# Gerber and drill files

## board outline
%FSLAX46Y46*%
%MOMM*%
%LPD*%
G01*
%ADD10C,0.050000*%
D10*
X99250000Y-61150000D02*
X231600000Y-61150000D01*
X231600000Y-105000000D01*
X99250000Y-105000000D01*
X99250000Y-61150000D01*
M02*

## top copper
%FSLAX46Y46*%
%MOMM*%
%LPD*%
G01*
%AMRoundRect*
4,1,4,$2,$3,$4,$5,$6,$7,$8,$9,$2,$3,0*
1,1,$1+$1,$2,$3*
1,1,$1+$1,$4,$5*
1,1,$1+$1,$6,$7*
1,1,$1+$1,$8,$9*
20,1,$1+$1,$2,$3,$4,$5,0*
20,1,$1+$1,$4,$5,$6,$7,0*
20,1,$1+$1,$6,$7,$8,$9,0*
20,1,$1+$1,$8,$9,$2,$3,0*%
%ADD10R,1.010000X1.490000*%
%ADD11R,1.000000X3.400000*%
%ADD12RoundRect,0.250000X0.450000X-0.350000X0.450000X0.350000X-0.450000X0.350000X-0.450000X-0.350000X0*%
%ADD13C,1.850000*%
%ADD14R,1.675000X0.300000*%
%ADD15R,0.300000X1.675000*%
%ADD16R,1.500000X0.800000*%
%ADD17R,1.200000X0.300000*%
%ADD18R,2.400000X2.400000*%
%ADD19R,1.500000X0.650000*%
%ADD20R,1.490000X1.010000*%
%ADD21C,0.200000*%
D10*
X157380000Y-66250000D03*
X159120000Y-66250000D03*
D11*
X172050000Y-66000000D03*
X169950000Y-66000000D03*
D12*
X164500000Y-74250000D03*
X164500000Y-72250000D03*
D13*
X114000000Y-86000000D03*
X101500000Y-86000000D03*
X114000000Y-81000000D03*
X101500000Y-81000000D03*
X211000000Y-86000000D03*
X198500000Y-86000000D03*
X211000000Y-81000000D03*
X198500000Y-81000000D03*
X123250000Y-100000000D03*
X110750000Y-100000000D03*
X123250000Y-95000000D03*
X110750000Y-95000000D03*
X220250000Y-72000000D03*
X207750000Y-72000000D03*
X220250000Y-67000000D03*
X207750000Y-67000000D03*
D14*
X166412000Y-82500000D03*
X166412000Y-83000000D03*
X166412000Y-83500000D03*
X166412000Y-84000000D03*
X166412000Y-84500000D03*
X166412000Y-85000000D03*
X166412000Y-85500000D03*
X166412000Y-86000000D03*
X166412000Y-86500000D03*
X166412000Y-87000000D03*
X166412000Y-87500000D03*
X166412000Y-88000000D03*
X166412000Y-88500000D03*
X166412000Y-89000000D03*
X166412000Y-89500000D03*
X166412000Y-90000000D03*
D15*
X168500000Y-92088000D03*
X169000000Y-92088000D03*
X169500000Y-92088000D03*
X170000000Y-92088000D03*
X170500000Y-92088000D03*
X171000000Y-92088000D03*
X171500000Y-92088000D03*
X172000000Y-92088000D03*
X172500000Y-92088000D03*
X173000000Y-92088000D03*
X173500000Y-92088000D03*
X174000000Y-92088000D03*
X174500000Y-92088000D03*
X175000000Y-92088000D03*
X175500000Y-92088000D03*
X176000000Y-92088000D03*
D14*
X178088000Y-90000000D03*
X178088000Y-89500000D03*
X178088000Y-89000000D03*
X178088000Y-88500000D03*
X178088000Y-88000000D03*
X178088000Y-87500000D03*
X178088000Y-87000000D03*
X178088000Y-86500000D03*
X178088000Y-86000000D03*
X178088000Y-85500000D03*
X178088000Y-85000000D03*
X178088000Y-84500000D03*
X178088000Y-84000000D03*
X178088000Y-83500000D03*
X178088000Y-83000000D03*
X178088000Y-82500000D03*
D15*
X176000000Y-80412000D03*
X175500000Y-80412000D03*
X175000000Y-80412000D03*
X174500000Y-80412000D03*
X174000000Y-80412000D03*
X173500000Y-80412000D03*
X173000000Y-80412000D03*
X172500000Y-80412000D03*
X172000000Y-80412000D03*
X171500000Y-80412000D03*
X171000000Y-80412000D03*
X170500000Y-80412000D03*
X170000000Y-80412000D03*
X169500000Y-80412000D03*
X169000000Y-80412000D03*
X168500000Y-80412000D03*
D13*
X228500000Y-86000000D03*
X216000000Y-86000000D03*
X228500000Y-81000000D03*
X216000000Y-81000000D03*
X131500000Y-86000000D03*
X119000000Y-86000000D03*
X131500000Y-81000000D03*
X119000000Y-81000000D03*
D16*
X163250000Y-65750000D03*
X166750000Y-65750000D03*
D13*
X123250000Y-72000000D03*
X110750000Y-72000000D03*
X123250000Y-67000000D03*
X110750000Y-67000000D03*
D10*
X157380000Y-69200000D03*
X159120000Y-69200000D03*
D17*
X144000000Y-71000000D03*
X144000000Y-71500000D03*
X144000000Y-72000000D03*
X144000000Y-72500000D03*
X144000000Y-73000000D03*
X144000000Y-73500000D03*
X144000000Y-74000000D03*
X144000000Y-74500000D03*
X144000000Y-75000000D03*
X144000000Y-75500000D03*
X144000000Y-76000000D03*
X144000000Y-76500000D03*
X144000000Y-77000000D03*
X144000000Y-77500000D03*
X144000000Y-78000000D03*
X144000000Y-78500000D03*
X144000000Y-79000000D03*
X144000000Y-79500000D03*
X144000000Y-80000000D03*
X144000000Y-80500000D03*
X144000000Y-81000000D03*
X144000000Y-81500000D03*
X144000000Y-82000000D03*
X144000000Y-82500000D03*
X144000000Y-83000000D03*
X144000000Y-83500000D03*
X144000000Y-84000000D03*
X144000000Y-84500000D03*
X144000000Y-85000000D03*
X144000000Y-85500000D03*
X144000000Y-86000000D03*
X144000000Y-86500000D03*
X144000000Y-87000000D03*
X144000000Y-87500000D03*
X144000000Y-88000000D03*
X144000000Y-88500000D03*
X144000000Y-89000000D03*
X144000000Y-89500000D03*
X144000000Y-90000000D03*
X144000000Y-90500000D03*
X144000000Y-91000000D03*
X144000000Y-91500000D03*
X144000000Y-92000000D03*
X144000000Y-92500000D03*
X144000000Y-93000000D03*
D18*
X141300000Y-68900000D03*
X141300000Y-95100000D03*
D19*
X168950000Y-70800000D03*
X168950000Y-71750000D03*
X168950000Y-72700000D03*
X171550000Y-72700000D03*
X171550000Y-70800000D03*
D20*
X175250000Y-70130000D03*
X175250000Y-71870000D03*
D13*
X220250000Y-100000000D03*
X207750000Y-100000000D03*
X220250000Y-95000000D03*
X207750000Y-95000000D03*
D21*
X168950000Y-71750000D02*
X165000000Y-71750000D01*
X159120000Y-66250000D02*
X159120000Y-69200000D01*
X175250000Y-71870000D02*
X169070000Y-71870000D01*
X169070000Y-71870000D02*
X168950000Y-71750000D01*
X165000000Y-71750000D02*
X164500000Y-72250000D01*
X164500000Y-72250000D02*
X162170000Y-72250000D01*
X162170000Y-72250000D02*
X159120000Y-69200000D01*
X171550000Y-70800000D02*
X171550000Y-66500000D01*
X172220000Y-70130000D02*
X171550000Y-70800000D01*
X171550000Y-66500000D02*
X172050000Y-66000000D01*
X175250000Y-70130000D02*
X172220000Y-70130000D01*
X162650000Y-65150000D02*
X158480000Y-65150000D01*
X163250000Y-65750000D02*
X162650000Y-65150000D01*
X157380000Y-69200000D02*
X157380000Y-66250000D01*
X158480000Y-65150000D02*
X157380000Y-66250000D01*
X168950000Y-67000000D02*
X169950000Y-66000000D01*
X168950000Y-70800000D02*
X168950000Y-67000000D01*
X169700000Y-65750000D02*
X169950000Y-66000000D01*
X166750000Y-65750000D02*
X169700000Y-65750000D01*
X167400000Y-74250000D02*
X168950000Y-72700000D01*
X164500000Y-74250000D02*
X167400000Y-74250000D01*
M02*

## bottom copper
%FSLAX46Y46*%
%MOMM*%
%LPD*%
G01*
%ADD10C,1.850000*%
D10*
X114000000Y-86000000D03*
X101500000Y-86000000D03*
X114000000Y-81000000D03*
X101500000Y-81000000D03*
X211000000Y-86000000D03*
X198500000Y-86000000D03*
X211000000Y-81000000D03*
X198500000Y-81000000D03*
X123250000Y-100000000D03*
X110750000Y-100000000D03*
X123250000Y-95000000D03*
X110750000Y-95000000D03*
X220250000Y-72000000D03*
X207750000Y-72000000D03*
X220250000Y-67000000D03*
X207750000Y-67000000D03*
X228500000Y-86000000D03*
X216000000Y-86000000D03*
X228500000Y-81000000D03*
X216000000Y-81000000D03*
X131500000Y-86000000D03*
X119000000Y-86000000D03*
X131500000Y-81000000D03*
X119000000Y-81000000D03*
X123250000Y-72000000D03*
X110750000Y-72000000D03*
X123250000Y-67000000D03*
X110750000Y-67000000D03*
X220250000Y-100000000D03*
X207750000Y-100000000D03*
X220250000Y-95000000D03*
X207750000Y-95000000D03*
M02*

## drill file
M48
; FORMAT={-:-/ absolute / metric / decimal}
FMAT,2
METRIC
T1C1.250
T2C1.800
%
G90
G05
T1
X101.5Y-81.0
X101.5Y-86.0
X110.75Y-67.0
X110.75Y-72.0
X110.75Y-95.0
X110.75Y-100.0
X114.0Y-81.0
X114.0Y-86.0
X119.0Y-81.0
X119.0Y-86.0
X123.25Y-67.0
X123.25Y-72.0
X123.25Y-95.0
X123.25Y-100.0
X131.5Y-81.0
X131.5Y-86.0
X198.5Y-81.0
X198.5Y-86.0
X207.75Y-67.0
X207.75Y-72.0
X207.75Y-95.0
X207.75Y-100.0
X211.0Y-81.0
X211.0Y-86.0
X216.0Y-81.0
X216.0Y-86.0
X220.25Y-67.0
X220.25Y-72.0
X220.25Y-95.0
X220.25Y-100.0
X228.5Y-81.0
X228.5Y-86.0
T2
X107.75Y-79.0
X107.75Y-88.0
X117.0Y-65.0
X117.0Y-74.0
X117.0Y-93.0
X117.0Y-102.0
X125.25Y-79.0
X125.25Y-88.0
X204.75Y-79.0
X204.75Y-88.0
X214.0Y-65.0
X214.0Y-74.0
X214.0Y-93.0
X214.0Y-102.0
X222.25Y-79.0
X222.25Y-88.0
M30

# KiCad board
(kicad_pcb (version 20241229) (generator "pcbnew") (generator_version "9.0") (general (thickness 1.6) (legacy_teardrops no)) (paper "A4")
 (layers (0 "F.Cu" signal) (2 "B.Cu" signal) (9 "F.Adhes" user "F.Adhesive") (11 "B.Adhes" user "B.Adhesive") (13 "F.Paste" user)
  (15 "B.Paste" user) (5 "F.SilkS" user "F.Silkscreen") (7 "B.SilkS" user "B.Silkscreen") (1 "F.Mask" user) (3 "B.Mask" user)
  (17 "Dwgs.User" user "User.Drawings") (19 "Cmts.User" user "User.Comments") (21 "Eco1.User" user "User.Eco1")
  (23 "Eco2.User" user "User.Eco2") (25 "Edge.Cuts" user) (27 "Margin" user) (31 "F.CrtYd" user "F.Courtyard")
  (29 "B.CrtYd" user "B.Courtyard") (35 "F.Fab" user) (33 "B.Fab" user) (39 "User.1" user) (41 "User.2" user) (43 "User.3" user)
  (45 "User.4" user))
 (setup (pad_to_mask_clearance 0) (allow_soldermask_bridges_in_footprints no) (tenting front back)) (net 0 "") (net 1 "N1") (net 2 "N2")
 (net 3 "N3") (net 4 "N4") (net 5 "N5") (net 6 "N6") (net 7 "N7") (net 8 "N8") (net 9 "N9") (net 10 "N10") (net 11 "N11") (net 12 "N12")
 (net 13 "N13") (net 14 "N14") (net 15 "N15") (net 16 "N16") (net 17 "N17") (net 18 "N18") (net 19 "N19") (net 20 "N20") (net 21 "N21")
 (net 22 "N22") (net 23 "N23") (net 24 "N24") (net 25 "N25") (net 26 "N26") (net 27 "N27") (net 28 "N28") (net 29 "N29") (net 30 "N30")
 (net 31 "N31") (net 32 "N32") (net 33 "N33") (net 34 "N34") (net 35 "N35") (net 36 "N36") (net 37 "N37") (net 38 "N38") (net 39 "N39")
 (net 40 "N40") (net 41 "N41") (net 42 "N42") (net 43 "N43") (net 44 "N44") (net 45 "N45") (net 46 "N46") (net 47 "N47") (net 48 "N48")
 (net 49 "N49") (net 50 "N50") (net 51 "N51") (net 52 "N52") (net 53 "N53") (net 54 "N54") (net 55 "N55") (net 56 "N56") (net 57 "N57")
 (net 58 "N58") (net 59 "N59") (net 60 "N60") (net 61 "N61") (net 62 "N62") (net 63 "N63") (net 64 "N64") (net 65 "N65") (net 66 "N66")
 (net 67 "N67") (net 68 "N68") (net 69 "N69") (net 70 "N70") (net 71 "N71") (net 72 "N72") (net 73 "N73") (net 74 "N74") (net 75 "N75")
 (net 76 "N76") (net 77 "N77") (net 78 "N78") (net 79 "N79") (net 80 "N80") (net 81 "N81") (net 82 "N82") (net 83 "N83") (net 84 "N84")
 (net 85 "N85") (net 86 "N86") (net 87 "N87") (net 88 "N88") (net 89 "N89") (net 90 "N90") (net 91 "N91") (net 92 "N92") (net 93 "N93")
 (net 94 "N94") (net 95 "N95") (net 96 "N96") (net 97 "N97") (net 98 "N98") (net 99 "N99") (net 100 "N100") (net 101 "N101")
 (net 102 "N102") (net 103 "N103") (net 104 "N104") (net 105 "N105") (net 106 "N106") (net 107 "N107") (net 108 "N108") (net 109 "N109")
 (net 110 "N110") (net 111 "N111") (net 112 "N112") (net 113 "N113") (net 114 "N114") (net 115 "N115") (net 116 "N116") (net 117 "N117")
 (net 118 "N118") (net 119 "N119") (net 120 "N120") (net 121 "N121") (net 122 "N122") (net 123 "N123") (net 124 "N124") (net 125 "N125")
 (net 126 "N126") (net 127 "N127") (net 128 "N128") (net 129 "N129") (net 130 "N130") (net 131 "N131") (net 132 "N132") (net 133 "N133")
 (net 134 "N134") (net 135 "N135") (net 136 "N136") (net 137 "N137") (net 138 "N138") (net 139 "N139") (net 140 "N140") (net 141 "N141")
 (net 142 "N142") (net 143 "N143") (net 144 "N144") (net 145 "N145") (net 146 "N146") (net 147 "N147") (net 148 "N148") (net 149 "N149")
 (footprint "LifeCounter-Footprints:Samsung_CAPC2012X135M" (layer "F.Cu") (at 158.25 66.25)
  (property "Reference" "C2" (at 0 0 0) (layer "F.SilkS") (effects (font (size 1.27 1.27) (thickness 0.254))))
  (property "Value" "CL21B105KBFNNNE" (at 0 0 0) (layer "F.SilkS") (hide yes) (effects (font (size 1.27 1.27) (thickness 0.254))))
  (pad "1" smd rect (at -0.87 0) (size 1.01 1.49) (layers "F.Cu" "F.Mask" "F.Paste") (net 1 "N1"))
  (pad "2" smd rect (at 0.87 0) (size 1.01 1.49) (layers "F.Cu" "F.Mask" "F.Paste") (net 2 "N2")))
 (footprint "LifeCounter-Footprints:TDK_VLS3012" (layer "F.Cu") (at 171 66 180)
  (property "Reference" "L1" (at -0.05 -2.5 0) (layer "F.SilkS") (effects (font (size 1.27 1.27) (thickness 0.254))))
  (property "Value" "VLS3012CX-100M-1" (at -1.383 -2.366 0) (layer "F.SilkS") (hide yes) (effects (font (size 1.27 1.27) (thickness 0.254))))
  (pad "1" smd rect (at -1.05 0 180) (size 1 3.4) (layers "F.Cu" "F.Mask" "F.Paste") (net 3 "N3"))
  (pad "2" smd rect (at 1.05 0 180) (size 1 3.4) (layers "F.Cu" "F.Mask" "F.Paste") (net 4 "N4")))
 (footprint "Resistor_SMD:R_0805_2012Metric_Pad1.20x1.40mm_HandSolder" (layer "F.Cu") (at 164.5 73.25 90)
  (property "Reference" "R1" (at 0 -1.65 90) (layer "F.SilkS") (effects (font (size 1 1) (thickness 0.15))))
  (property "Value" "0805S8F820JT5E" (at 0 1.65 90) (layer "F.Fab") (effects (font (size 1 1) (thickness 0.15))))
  (pad "1" smd roundrect (at -1 0 90) (size 1.2 1.4) (layers "F.Cu" "F.Mask" "F.Paste") (roundrect_rratio 0.208333) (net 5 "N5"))
  (pad "2" smd roundrect (at 1 0 90) (size 1.2 1.4) (layers "F.Cu" "F.Mask" "F.Paste") (roundrect_rratio 0.208333) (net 2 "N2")))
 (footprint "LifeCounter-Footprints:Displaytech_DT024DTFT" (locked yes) (layer "F.Cu") (at 143 83 -90)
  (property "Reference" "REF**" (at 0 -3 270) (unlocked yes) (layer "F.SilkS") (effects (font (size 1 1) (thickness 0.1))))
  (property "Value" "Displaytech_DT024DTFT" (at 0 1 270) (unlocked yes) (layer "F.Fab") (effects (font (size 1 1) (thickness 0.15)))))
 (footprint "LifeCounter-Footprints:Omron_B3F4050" (layer "F.Cu") (at 107.75 83.5)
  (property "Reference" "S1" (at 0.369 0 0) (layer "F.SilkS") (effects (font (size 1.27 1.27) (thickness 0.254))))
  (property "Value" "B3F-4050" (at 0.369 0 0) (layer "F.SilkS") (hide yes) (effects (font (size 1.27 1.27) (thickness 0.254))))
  (pad "" np_thru_hole circle (at 0 -4.5) (size 1.8 1.8) (drill 1.8) (layers "*.Cu" "*.Mask"))
  (pad "" np_thru_hole circle (at 0 4.5) (size 1.8 1.8) (drill 1.8) (layers "*.Cu" "*.Mask"))
  (pad "1" thru_hole circle (at 6.25 2.5) (size 1.85 1.85) (drill 1.25) (layers "*.Cu" "*.Mask") (remove_unused_layers no) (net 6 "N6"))
  (pad "2" thru_hole circle (at -6.25 2.5) (size 1.85 1.85) (drill 1.25) (layers "*.Cu" "*.Mask") (remove_unused_layers no) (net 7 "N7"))
  (pad "3" thru_hole circle (at 6.25 -2.5) (size 1.85 1.85) (drill 1.25) (layers "*.Cu" "*.Mask") (remove_unused_layers no) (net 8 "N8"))
  (pad "4" thru_hole circle (at -6.25 -2.5) (size 1.85 1.85) (drill 1.25) (layers "*.Cu" "*.Mask") (remove_unused_layers no) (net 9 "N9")))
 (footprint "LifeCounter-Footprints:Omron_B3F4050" (layer "F.Cu") (at 204.75 83.5)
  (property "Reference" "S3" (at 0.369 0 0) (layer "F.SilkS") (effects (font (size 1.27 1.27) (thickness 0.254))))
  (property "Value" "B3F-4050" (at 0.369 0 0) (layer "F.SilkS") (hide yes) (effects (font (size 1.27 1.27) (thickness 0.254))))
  (pad "" np_thru_hole circle (at 0 -4.5) (size 1.8 1.8) (drill 1.8) (layers "*.Cu" "*.Mask"))
  (pad "" np_thru_hole circle (at 0 4.5) (size 1.8 1.8) (drill 1.8) (layers "*.Cu" "*.Mask"))
  (pad "1" thru_hole circle (at 6.25 2.5) (size 1.85 1.85) (drill 1.25) (layers "*.Cu" "*.Mask") (remove_unused_layers no) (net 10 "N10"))
  (pad "2" thru_hole circle (at -6.25 2.5) (size 1.85 1.85) (drill 1.25) (layers "*.Cu" "*.Mask") (remove_unused_layers no) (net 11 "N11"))
  (pad "3" thru_hole circle (at 6.25 -2.5) (size 1.85 1.85) (drill 1.25) (layers "*.Cu" "*.Mask") (remove_unused_layers no) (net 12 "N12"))
  (pad "4" thru_hole circle (at -6.25 -2.5) (size 1.85 1.85) (drill 1.25) (layers "*.Cu" "*.Mask") (remove_unused_layers no) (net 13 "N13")))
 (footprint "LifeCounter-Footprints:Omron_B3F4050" (layer "F.Cu") (at 117 97.5)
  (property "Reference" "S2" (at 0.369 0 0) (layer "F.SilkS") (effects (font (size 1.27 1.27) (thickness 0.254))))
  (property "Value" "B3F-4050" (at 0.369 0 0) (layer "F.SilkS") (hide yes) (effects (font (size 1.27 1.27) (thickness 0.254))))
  (pad "" np_thru_hole circle (at 0 -4.5) (size 1.8 1.8) (drill 1.8) (layers "*.Cu" "*.Mask"))
  (pad "" np_thru_hole circle (at 0 4.5) (size 1.8 1.8) (drill 1.8) (layers "*.Cu" "*.Mask"))
  (pad "1" thru_hole circle (at 6.25 2.5) (size 1.85 1.85) (drill 1.25) (layers "*.Cu" "*.Mask") (remove_unused_layers no) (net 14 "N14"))
  (pad "2" thru_hole circle (at -6.25 2.5) (size 1.85 1.85) (drill 1.25) (layers "*.Cu" "*.Mask") (remove_unused_layers no) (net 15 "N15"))
  (pad "3" thru_hole circle (at 6.25 -2.5) (size 1.85 1.85) (drill 1.25) (layers "*.Cu" "*.Mask") (remove_unused_layers no) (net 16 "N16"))
  (pad "4" thru_hole circle (at -6.25 -2.5) (size 1.85 1.85) (drill 1.25) (layers "*.Cu" "*.Mask") (remove_unused_layers no) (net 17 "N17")))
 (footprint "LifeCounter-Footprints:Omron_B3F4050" (layer "F.Cu") (at 214 69.5)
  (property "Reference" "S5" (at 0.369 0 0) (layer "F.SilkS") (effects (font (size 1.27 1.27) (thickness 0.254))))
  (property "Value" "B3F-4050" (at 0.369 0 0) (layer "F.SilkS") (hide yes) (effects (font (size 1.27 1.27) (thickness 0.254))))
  (pad "" np_thru_hole circle (at 0 -4.5) (size 1.8 1.8) (drill 1.8) (layers "*.Cu" "*.Mask"))
  (pad "" np_thru_hole circle (at 0 4.5) (size 1.8 1.8) (drill 1.8) (layers "*.Cu" "*.Mask"))
  (pad "1" thru_hole circle (at 6.25 2.5) (size 1.85 1.85) (drill 1.25) (layers "*.Cu" "*.Mask") (remove_unused_layers no) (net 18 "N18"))
  (pad "2" thru_hole circle (at -6.25 2.5) (size 1.85 1.85) (drill 1.25) (layers "*.Cu" "*.Mask") (remove_unused_layers no) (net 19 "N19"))
  (pad "3" thru_hole circle (at 6.25 -2.5) (size 1.85 1.85) (drill 1.25) (layers "*.Cu" "*.Mask") (remove_unused_layers no) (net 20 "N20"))
  (pad "4" thru_hole circle (at -6.25 -2.5) (size 1.85 1.85) (drill 1.25) (layers "*.Cu" "*.Mask") (remove_unused_layers no) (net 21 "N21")))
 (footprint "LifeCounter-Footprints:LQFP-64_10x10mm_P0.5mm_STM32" (layer "F.Cu") (at 172.25 86.25)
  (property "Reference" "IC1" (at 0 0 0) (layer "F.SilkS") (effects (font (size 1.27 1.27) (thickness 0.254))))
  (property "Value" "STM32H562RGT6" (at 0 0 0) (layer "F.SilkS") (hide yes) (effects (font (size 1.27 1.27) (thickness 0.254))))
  (pad "1" smd rect (at -5.838 -3.75 90) (size 0.3 1.675) (layers "F.Cu" "F.Mask" "F.Paste") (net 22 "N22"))
  (pad "2" smd rect (at -5.838 -3.25 90) (size 0.3 1.675) (layers "F.Cu" "F.Mask" "F.Paste") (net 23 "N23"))
  (pad "3" smd rect (at -5.838 -2.75 90) (size 0.3 1.675) (layers "F.Cu" "F.Mask" "F.Paste") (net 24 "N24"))
  (pad "4" smd rect (at -5.838 -2.25 90) (size 0.3 1.675) (layers "F.Cu" "F.Mask" "F.Paste") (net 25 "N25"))
  (pad "5" smd rect (at -5.838 -1.75 90) (size 0.3 1.675) (layers "F.Cu" "F.Mask" "F.Paste") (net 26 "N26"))
  (pad "6" smd rect (at -5.838 -1.25 90) (size 0.3 1.675) (layers "F.Cu" "F.Mask" "F.Paste") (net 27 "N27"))
  (pad "7" smd rect (at -5.838 -0.75 90) (size 0.3 1.675) (layers "F.Cu" "F.Mask" "F.Paste") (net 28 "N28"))
  (pad "8" smd rect (at -5.838 -0.25 90) (size 0.3 1.675) (layers "F.Cu" "F.Mask" "F.Paste") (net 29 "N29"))
  (pad "9" smd rect (at -5.838 0.25 90) (size 0.3 1.675) (layers "F.Cu" "F.Mask" "F.Paste") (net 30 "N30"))
  (pad "10" smd rect (at -5.838 0.75 90) (size 0.3 1.675) (layers "F.Cu" "F.Mask" "F.Paste") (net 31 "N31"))
  (pad "11" smd rect (at -5.838 1.25 90) (size 0.3 1.675) (layers "F.Cu" "F.Mask" "F.Paste") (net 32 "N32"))
  (pad "12" smd rect (at -5.838 1.75 90) (size 0.3 1.675) (layers "F.Cu" "F.Mask" "F.Paste") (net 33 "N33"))
  (pad "13" smd rect (at -5.838 2.25 90) (size 0.3 1.675) (layers "F.Cu" "F.Mask" "F.Paste") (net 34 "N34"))
  (pad "14" smd rect (at -5.838 2.75 90) (size 0.3 1.675) (layers "F.Cu" "F.Mask" "F.Paste") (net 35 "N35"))
  (pad "15" smd rect (at -5.838 3.25 90) (size 0.3 1.675) (layers "F.Cu" "F.Mask" "F.Paste") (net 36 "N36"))
  (pad "16" smd rect (at -5.838 3.75 90) (size 0.3 1.675) (layers "F.Cu" "F.Mask" "F.Paste") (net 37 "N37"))
  (pad "17" smd rect (at -3.75 5.838) (size 0.3 1.675) (layers "F.Cu" "F.Mask" "F.Paste") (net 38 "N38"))
  (pad "18" smd rect (at -3.25 5.838) (size 0.3 1.675) (layers "F.Cu" "F.Mask" "F.Paste") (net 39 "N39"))
  (pad "19" smd rect (at -2.75 5.838) (size 0.3 1.675) (layers "F.Cu" "F.Mask" "F.Paste") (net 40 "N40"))
  (pad "20" smd rect (at -2.25 5.838) (size 0.3 1.675) (layers "F.Cu" "F.Mask" "F.Paste") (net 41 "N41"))
  (pad "21" smd rect (at -1.75 5.838) (size 0.3 1.675) (layers "F.Cu" "F.Mask" "F.Paste") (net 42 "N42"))
  (pad "22" smd rect (at -1.25 5.838) (size 0.3 1.675) (layers "F.Cu" "F.Mask" "F.Paste") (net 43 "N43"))
  (pad "23" smd rect (at -0.75 5.838) (size 0.3 1.675) (layers "F.Cu" "F.Mask" "F.Paste") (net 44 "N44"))
  (pad "24" smd rect (at -0.25 5.838) (size 0.3 1.675) (layers "F.Cu" "F.Mask" "F.Paste") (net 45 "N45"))
  (pad "25" smd rect (at 0.25 5.838) (size 0.3 1.675) (layers "F.Cu" "F.Mask" "F.Paste") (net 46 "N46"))
  (pad "26" smd rect (at 0.75 5.838) (size 0.3 1.675) (layers "F.Cu" "F.Mask" "F.Paste") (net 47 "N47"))
  (pad "27" smd rect (at 1.25 5.838) (size 0.3 1.675) (layers "F.Cu" "F.Mask" "F.Paste") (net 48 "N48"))
  (pad "28" smd rect (at 1.75 5.838) (size 0.3 1.675) (layers "F.Cu" "F.Mask" "F.Paste") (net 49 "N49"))
  (pad "29" smd rect (at 2.25 5.838) (size 0.3 1.675) (layers "F.Cu" "F.Mask" "F.Paste") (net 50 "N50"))
  (pad "30" smd rect (at 2.75 5.838) (size 0.3 1.675) (layers "F.Cu" "F.Mask" "F.Paste") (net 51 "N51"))
  (pad "31" smd rect (at 3.25 5.838) (size 0.3 1.675) (layers "F.Cu" "F.Mask" "F.Paste") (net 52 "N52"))
  (pad "32" smd rect (at 3.75 5.838) (size 0.3 1.675) (layers "F.Cu" "F.Mask" "F.Paste") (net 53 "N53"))
  (pad "33" smd rect (at 5.838 3.75 90) (size 0.3 1.675) (layers "F.Cu" "F.Mask" "F.Paste") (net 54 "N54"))
  (pad "34" smd rect (at 5.838 3.25 90) (size 0.3 1.675) (layers "F.Cu" "F.Mask" "F.Paste") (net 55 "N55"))
  (pad "35" smd rect (at 5.838 2.75 90) (size 0.3 1.675) (layers "F.Cu" "F.Mask" "F.Paste") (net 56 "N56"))
  (pad "36" smd rect (at 5.838 2.25 90) (size 0.3 1.675) (layers "F.Cu" "F.Mask" "F.Paste") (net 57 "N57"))
  (pad "37" smd rect (at 5.838 1.75 90) (size 0.3 1.675) (layers "F.Cu" "F.Mask" "F.Paste") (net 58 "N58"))
  (pad "38" smd rect (at 5.838 1.25 90) (size 0.3 1.675) (layers "F.Cu" "F.Mask" "F.Paste") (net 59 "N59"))
  (pad "39" smd rect (at 5.838 0.75 90) (size 0.3 1.675) (layers "F.Cu" "F.Mask" "F.Paste") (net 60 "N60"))
  (pad "40" smd rect (at 5.838 0.25 90) (size 0.3 1.675) (layers "F.Cu" "F.Mask" "F.Paste") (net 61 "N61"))
  (pad "41" smd rect (at 5.838 -0.25 90) (size 0.3 1.675) (layers "F.Cu" "F.Mask" "F.Paste") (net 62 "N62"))
  (pad "42" smd rect (at 5.838 -0.75 90) (size 0.3 1.675) (layers "F.Cu" "F.Mask" "F.Paste") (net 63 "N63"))
  (pad "43" smd rect (at 5.838 -1.25 90) (size 0.3 1.675) (layers "F.Cu" "F.Mask" "F.Paste") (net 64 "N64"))
  (pad "44" smd rect (at 5.838 -1.75 90) (size 0.3 1.675) (layers "F.Cu" "F.Mask" "F.Paste") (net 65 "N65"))
  (pad "45" smd rect (at 5.838 -2.25 90) (size 0.3 1.675) (layers "F.Cu" "F.Mask" "F.Paste") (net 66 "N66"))
  (pad "46" smd rect (at 5.838 -2.75 90) (size 0.3 1.675) (layers "F.Cu" "F.Mask" "F.Paste") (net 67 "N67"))
  (pad "47" smd rect (at 5.838 -3.25 90) (size 0.3 1.675) (layers "F.Cu" "F.Mask" "F.Paste") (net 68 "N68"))
  (pad "48" smd rect (at 5.838 -3.75 90) (size 0.3 1.675) (layers "F.Cu" "F.Mask" "F.Paste") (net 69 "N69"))
  (pad "49" smd rect (at 3.75 -5.838) (size 0.3 1.675) (layers "F.Cu" "F.Mask" "F.Paste") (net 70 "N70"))
  (pad "50" smd rect (at 3.25 -5.838) (size 0.3 1.675) (layers "F.Cu" "F.Mask" "F.Paste") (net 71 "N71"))
  (pad "51" smd rect (at 2.75 -5.838) (size 0.3 1.675) (layers "F.Cu" "F.Mask" "F.Paste") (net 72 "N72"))
  (pad "52" smd rect (at 2.25 -5.838) (size 0.3 1.675) (layers "F.Cu" "F.Mask" "F.Paste") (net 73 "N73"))
  (pad "53" smd rect (at 1.75 -5.838) (size 0.3 1.675) (layers "F.Cu" "F.Mask" "F.Paste") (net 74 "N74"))
  (pad "54" smd rect (at 1.25 -5.838) (size 0.3 1.675) (layers "F.Cu" "F.Mask" "F.Paste") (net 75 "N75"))
  (pad "55" smd rect (at 0.75 -5.838) (size 0.3 1.675) (layers "F.Cu" "F.Mask" "F.Paste") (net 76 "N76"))
  (pad "56" smd rect (at 0.25 -5.838) (size 0.3 1.675) (layers "F.Cu" "F.Mask" "F.Paste") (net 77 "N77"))
  (pad "57" smd rect (at -0.25 -5.838) (size 0.3 1.675) (layers "F.Cu" "F.Mask" "F.Paste") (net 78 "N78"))
  (pad "58" smd rect (at -0.75 -5.838) (size 0.3 1.675) (layers "F.Cu" "F.Mask" "F.Paste") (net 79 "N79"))
  (pad "59" smd rect (at -1.25 -5.838) (size 0.3 1.675) (layers "F.Cu" "F.Mask" "F.Paste") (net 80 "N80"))
  (pad "60" smd rect (at -1.75 -5.838) (size 0.3 1.675) (layers "F.Cu" "F.Mask" "F.Paste") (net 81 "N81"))
  (pad "61" smd rect (at -2.25 -5.838) (size 0.3 1.675) (layers "F.Cu" "F.Mask" "F.Paste") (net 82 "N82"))
  (pad "62" smd rect (at -2.75 -5.838) (size 0.3 1.675) (layers "F.Cu" "F.Mask" "F.Paste") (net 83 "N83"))
  (pad "63" smd rect (at -3.25 -5.838) (size 0.3 1.675) (layers "F.Cu" "F.Mask" "F.Paste") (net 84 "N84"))
  (pad "64" smd rect (at -3.75 -5.838) (size 0.3 1.675) (layers "F.Cu" "F.Mask" "F.Paste") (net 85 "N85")))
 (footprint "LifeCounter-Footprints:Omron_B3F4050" (layer "F.Cu") (at 222.25 83.5)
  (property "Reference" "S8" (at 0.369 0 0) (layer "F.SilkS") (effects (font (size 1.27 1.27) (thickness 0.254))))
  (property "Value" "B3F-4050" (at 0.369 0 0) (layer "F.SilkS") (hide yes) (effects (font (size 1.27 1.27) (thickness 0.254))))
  (pad "" np_thru_hole circle (at 0 -4.5) (size 1.8 1.8) (drill 1.8) (layers "*.Cu" "*.Mask"))
  (pad "" np_thru_hole circle (at 0 4.5) (size 1.8 1.8) (drill 1.8) (layers "*.Cu" "*.Mask"))
  (pad "1" thru_hole circle (at 6.25 2.5) (size 1.85 1.85) (drill 1.25) (layers "*.Cu" "*.Mask") (remove_unused_layers no) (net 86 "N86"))
  (pad "2" thru_hole circle (at -6.25 2.5) (size 1.85 1.85) (drill 1.25) (layers "*.Cu" "*.Mask") (remove_unused_layers no) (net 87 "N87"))
  (pad "3" thru_hole circle (at 6.25 -2.5) (size 1.85 1.85) (drill 1.25) (layers "*.Cu" "*.Mask") (remove_unused_layers no) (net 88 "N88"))
  (pad "4" thru_hole circle (at -6.25 -2.5) (size 1.85 1.85) (drill 1.25) (layers "*.Cu" "*.Mask") (remove_unused_layers no) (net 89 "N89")))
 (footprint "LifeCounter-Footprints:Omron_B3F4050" (layer "F.Cu") (at 125.25 83.5)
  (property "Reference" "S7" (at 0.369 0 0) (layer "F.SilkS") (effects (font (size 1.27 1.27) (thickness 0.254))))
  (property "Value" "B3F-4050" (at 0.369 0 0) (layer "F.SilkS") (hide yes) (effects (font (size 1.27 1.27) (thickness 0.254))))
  (pad "" np_thru_hole circle (at 0 -4.5) (size 1.8 1.8) (drill 1.8) (layers "*.Cu" "*.Mask"))
  (pad "" np_thru_hole circle (at 0 4.5) (size 1.8 1.8) (drill 1.8) (layers "*.Cu" "*.Mask"))
  (pad "1" thru_hole circle (at 6.25 2.5) (size 1.85 1.85) (drill 1.25) (layers "*.Cu" "*.Mask") (remove_unused_layers no) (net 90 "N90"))
  (pad "2" thru_hole circle (at -6.25 2.5) (size 1.85 1.85) (drill 1.25) (layers "*.Cu" "*.Mask") (remove_unused_layers no) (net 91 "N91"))
  (pad "3" thru_hole circle (at 6.25 -2.5) (size 1.85 1.85) (drill 1.25) (layers "*.Cu" "*.Mask") (remove_unused_layers no) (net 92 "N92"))
  (pad "4" thru_hole circle (at -6.25 -2.5) (size 1.85 1.85) (drill 1.25) (layers "*.Cu" "*.Mask") (remove_unused_layers no) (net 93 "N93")))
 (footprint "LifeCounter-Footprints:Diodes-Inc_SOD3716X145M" (layer "F.Cu") (at 165 65.75)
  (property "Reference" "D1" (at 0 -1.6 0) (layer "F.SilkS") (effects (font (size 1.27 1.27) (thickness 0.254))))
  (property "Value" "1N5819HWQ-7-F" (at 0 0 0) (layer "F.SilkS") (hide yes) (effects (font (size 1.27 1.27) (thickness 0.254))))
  (pad "1" smd rect (at -1.75 0 90) (size 0.8 1.5) (layers "F.Cu" "F.Mask" "F.Paste") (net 1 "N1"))
  (pad "2" smd rect (at 1.75 0 90) (size 0.8 1.5) (layers "F.Cu" "F.Mask" "F.Paste") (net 4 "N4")))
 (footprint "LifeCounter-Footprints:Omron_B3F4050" (layer "F.Cu") (at 117 69.5)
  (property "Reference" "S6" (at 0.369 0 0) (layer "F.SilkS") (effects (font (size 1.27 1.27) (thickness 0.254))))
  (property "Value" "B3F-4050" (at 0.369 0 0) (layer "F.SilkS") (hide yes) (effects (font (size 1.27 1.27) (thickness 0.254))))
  (pad "" np_thru_hole circle (at 0 -4.5) (size 1.8 1.8) (drill 1.8) (layers "*.Cu" "*.Mask"))
  (pad "" np_thru_hole circle (at 0 4.5) (size 1.8 1.8) (drill 1.8) (layers "*.Cu" "*.Mask"))
  (pad "1" thru_hole circle (at 6.25 2.5) (size 1.85 1.85) (drill 1.25) (layers "*.Cu" "*.Mask") (remove_unused_layers no) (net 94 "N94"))
  (pad "2" thru_hole circle (at -6.25 2.5) (size 1.85 1.85) (drill 1.25) (layers "*.Cu" "*.Mask") (remove_unused_layers no) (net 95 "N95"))
  (pad "3" thru_hole circle (at 6.25 -2.5) (size 1.85 1.85) (drill 1.25) (layers "*.Cu" "*.Mask") (remove_unused_layers no) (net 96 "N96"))
  (pad "4" thru_hole circle (at -6.25 -2.5) (size 1.85 1.85) (drill 1.25) (layers "*.Cu" "*.Mask") (remove_unused_layers no) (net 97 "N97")))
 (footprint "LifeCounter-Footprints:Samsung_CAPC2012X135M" (layer "F.Cu") (at 158.25 69.2)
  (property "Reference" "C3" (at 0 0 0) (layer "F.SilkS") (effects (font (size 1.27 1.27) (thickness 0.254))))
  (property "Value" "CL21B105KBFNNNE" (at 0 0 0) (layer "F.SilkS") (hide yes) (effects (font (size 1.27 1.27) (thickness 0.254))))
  (pad "1" smd rect (at -0.87 0) (size 1.01 1.49) (layers "F.Cu" "F.Mask" "F.Paste") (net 1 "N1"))
  (pad "2" smd rect (at 0.87 0) (size 1.01 1.49) (layers "F.Cu" "F.Mask" "F.Paste") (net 2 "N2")))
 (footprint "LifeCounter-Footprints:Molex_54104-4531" (layer "F.Cu") (at 140.425 82 -90)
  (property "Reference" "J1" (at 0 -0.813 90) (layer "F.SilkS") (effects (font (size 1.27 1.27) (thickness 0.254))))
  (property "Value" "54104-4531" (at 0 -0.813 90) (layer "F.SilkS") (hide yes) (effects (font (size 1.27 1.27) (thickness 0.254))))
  (pad "1" smd rect (at -11 -3.575 270) (size 0.3 1.2) (layers "F.Cu" "F.Mask" "F.Paste") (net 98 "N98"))
  (pad "2" smd rect (at -10.5 -3.575 270) (size 0.3 1.2) (layers "F.Cu" "F.Mask" "F.Paste") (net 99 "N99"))
  (pad "3" smd rect (at -10 -3.575 270) (size 0.3 1.2) (layers "F.Cu" "F.Mask" "F.Paste") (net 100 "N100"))
  (pad "4" smd rect (at -9.5 -3.575 270) (size 0.3 1.2) (layers "F.Cu" "F.Mask" "F.Paste") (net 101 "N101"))
  (pad "5" smd rect (at -9 -3.575 270) (size 0.3 1.2) (layers "F.Cu" "F.Mask" "F.Paste") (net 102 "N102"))
  (pad "6" smd rect (at -8.5 -3.575 270) (size 0.3 1.2) (layers "F.Cu" "F.Mask" "F.Paste") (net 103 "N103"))
  (pad "7" smd rect (at -8 -3.575 270) (size 0.3 1.2) (layers "F.Cu" "F.Mask" "F.Paste") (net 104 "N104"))
  (pad "8" smd rect (at -7.5 -3.575 270) (size 0.3 1.2) (layers "F.Cu" "F.Mask" "F.Paste") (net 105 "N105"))
  (pad "9" smd rect (at -7 -3.575 270) (size 0.3 1.2) (layers "F.Cu" "F.Mask" "F.Paste") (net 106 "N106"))
  (pad "10" smd rect (at -6.5 -3.575 270) (size 0.3 1.2) (layers "F.Cu" "F.Mask" "F.Paste") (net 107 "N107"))
  (pad "11" smd rect (at -6 -3.575 270) (size 0.3 1.2) (layers "F.Cu" "F.Mask" "F.Paste") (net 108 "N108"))
  (pad "12" smd rect (at -5.5 -3.575 270) (size 0.3 1.2) (layers "F.Cu" "F.Mask" "F.Paste") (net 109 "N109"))
  (pad "13" smd rect (at -5 -3.575 270) (size 0.3 1.2) (layers "F.Cu" "F.Mask" "F.Paste") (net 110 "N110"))
  (pad "14" smd rect (at -4.5 -3.575 270) (size 0.3 1.2) (layers "F.Cu" "F.Mask" "F.Paste") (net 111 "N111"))
  (pad "15" smd rect (at -4 -3.575 270) (size 0.3 1.2) (layers "F.Cu" "F.Mask" "F.Paste") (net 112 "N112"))
  (pad "16" smd rect (at -3.5 -3.575 270) (size 0.3 1.2) (layers "F.Cu" "F.Mask" "F.Paste") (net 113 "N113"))
  (pad "17" smd rect (at -3 -3.575 270) (size 0.3 1.2) (layers "F.Cu" "F.Mask" "F.Paste") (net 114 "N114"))
  (pad "18" smd rect (at -2.5 -3.575 270) (size 0.3 1.2) (layers "F.Cu" "F.Mask" "F.Paste") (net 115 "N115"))
  (pad "19" smd rect (at -2 -3.575 270) (size 0.3 1.2) (layers "F.Cu" "F.Mask" "F.Paste") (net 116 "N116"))
  (pad "20" smd rect (at -1.5 -3.575 270) (size 0.3 1.2) (layers "F.Cu" "F.Mask" "F.Paste") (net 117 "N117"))
  (pad "21" smd rect (at -1 -3.575 270) (size 0.3 1.2) (layers "F.Cu" "F.Mask" "F.Paste") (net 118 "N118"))
  (pad "22" smd rect (at -0.5 -3.575 270) (size 0.3 1.2) (layers "F.Cu" "F.Mask" "F.Paste") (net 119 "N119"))
  (pad "23" smd rect (at 0 -3.575 270) (size 0.3 1.2) (layers "F.Cu" "F.Mask" "F.Paste") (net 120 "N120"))
  (pad "24" smd rect (at 0.5 -3.575 270) (size 0.3 1.2) (layers "F.Cu" "F.Mask" "F.Paste") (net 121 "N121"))
  (pad "25" smd rect (at 1 -3.575 270) (size 0.3 1.2) (layers "F.Cu" "F.Mask" "F.Paste") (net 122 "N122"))
  (pad "26" smd rect (at 1.5 -3.575 270) (size 0.3 1.2) (layers "F.Cu" "F.Mask" "F.Paste") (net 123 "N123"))
  (pad "27" smd rect (at 2 -3.575 270) (size 0.3 1.2) (layers "F.Cu" "F.Mask" "F.Paste") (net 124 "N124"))
  (pad "28" smd rect (at 2.5 -3.575 270) (size 0.3 1.2) (layers "F.Cu" "F.Mask" "F.Paste") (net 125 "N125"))
  (pad "29" smd rect (at 3 -3.575 270) (size 0.3 1.2) (layers "F.Cu" "F.Mask" "F.Paste") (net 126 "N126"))
  (pad "30" smd rect (at 3.5 -3.575 270) (size 0.3 1.2) (layers "F.Cu" "F.Mask" "F.Paste") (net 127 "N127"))
  (pad "31" smd rect (at 4 -3.575 270) (size 0.3 1.2) (layers "F.Cu" "F.Mask" "F.Paste") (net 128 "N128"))
  (pad "32" smd rect (at 4.5 -3.575 270) (size 0.3 1.2) (layers "F.Cu" "F.Mask" "F.Paste") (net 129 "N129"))
  (pad "33" smd rect (at 5 -3.575 270) (size 0.3 1.2) (layers "F.Cu" "F.Mask" "F.Paste") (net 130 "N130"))
  (pad "34" smd rect (at 5.5 -3.575 270) (size 0.3 1.2) (layers "F.Cu" "F.Mask" "F.Paste") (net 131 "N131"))
  (pad "35" smd rect (at 6 -3.575 270) (size 0.3 1.2) (layers "F.Cu" "F.Mask" "F.Paste") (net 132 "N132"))
  (pad "36" smd rect (at 6.5 -3.575 270) (size 0.3 1.2) (layers "F.Cu" "F.Mask" "F.Paste") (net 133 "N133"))
  (pad "37" smd rect (at 7 -3.575 270) (size 0.3 1.2) (layers "F.Cu" "F.Mask" "F.Paste") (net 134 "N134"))
  (pad "38" smd rect (at 7.5 -3.575 270) (size 0.3 1.2) (layers "F.Cu" "F.Mask" "F.Paste") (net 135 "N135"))
  (pad "39" smd rect (at 8 -3.575 270) (size 0.3 1.2) (layers "F.Cu" "F.Mask" "F.Paste") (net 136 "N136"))
  (pad "40" smd rect (at 8.5 -3.575 270) (size 0.3 1.2) (layers "F.Cu" "F.Mask" "F.Paste") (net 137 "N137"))
  (pad "41" smd rect (at 9 -3.575 270) (size 0.3 1.2) (layers "F.Cu" "F.Mask" "F.Paste") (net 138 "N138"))
  (pad "42" smd rect (at 9.5 -3.575 270) (size 0.3 1.2) (layers "F.Cu" "F.Mask" "F.Paste") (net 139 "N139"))
  (pad "43" smd rect (at 10 -3.575 270) (size 0.3 1.2) (layers "F.Cu" "F.Mask" "F.Paste") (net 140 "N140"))
  (pad "44" smd rect (at 10.5 -3.575 270) (size 0.3 1.2) (layers "F.Cu" "F.Mask" "F.Paste") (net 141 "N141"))
  (pad "45" smd rect (at 11 -3.575 270) (size 0.3 1.2) (layers "F.Cu" "F.Mask" "F.Paste") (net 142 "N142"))
  (pad "MP1" smd rect (at -13.1 -0.875) (size 2.4 2.4) (layers "F.Cu" "F.Mask" "F.Paste") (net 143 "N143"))
  (pad "MP2" smd rect (at 13.1 -0.875) (size 2.4 2.4) (layers "F.Cu" "F.Mask" "F.Paste") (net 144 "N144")))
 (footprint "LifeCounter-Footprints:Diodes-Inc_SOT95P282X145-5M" (layer "F.Cu") (at 170.25 71.75)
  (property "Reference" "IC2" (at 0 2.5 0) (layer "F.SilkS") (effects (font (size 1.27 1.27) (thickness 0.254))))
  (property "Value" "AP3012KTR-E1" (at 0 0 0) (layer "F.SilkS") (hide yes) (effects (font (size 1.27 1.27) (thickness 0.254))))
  (pad "1" smd rect (at -1.3 -0.95 90) (size 0.65 1.5) (layers "F.Cu" "F.Mask" "F.Paste") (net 4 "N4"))
  (pad "2" smd rect (at -1.3 0 90) (size 0.65 1.5) (layers "F.Cu" "F.Mask" "F.Paste") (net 2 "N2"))
  (pad "3" smd rect (at -1.3 0.95 90) (size 0.65 1.5) (layers "F.Cu" "F.Mask" "F.Paste") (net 5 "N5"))
  (pad "4" smd rect (at 1.3 0.95 90) (size 0.65 1.5) (layers "F.Cu" "F.Mask" "F.Paste") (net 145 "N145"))
  (pad "5" smd rect (at 1.3 -0.95 90) (size 0.65 1.5) (layers "F.Cu" "F.Mask" "F.Paste") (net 3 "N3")))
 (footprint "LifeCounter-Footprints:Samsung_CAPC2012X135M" (layer "F.Cu") (at 175.25 71 -90)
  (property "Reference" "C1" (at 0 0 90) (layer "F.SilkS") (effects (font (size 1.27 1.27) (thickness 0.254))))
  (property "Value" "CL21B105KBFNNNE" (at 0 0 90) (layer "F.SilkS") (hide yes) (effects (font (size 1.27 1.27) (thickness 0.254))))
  (pad "1" smd rect (at -0.87 0 270) (size 1.01 1.49) (layers "F.Cu" "F.Mask" "F.Paste") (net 3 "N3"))
  (pad "2" smd rect (at 0.87 0 270) (size 1.01 1.49) (layers "F.Cu" "F.Mask" "F.Paste") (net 2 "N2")))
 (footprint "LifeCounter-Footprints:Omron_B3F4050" (layer "F.Cu") (at 214 97.5)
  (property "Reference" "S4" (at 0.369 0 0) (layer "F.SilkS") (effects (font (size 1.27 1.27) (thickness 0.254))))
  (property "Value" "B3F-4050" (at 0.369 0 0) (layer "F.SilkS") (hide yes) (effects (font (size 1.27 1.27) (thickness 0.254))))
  (pad "" np_thru_hole circle (at 0 -4.5) (size 1.8 1.8) (drill 1.8) (layers "*.Cu" "*.Mask"))
  (pad "" np_thru_hole circle (at 0 4.5) (size 1.8 1.8) (drill 1.8) (layers "*.Cu" "*.Mask"))
  (pad "1" thru_hole circle (at 6.25 2.5) (size 1.85 1.85) (drill 1.25) (layers "*.Cu" "*.Mask") (remove_unused_layers no) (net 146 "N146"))
  (pad "2" thru_hole circle (at -6.25 2.5) (size 1.85 1.85) (drill 1.25) (layers "*.Cu" "*.Mask") (remove_unused_layers no) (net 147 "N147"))
  (pad "3" thru_hole circle (at 6.25 -2.5) (size 1.85 1.85) (drill 1.25) (layers "*.Cu" "*.Mask") (remove_unused_layers no) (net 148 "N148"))
  (pad "4" thru_hole circle (at -6.25 -2.5) (size 1.85 1.85) (drill 1.25) (layers "*.Cu" "*.Mask") (remove_unused_layers no)
   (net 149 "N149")))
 (gr_rect (start 99.25 61.15) (end 231.6 105) (stroke (width 0.05) (type default)) (fill no) (layer "Edge.Cuts"))
 (segment (start 168.95 71.75) (end 165 71.75) (width 0.2) (layer "F.Cu") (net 2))
 (segment (start 159.12 66.25) (end 159.12 69.2) (width 0.2) (layer "F.Cu") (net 2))
 (segment (start 175.25 71.87) (end 169.07 71.87) (width 0.2) (layer "F.Cu") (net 2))
 (segment (start 169.07 71.87) (end 168.95 71.75) (width 0.2) (layer "F.Cu") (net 2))
 (segment (start 165 71.75) (end 164.5 72.25) (width 0.2) (layer "F.Cu") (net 2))
 (segment (start 164.5 72.25) (end 162.17 72.25) (width 0.2) (layer "F.Cu") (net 2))
 (segment (start 162.17 72.25) (end 159.12 69.2) (width 0.2) (layer "F.Cu") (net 2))
 (segment (start 171.55 70.8) (end 171.55 66.5) (width 0.2) (layer "F.Cu") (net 3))
 (segment (start 172.22 70.13) (end 171.55 70.8) (width 0.2) (layer "F.Cu") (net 3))
 (segment (start 171.55 66.5) (end 172.05 66) (width 0.2) (layer "F.Cu") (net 3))
 (segment (start 175.25 70.13) (end 172.22 70.13) (width 0.2) (layer "F.Cu") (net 3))
 (segment (start 162.65 65.15) (end 158.48 65.15) (width 0.2) (layer "F.Cu") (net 1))
 (segment (start 163.25 65.75) (end 162.65 65.15) (width 0.2) (layer "F.Cu") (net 1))
 (segment (start 157.38 69.2) (end 157.38 66.25) (width 0.2) (layer "F.Cu") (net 1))
 (segment (start 158.48 65.15) (end 157.38 66.25) (width 0.2) (layer "F.Cu") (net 1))
 (segment (start 168.95 67) (end 169.95 66) (width 0.2) (layer "F.Cu") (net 4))
 (segment (start 168.95 70.8) (end 168.95 67) (width 0.2) (layer "F.Cu") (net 4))
 (segment (start 169.7 65.75) (end 169.95 66) (width 0.2) (layer "F.Cu") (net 4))
 (segment (start 166.75 65.75) (end 169.7 65.75) (width 0.2) (layer "F.Cu") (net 4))
 (segment (start 167.4 74.25) (end 168.95 72.7) (width 0.2) (layer "F.Cu") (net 5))
 (segment (start 164.5 74.25) (end 167.4 74.25) (width 0.2) (layer "F.Cu") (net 5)))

